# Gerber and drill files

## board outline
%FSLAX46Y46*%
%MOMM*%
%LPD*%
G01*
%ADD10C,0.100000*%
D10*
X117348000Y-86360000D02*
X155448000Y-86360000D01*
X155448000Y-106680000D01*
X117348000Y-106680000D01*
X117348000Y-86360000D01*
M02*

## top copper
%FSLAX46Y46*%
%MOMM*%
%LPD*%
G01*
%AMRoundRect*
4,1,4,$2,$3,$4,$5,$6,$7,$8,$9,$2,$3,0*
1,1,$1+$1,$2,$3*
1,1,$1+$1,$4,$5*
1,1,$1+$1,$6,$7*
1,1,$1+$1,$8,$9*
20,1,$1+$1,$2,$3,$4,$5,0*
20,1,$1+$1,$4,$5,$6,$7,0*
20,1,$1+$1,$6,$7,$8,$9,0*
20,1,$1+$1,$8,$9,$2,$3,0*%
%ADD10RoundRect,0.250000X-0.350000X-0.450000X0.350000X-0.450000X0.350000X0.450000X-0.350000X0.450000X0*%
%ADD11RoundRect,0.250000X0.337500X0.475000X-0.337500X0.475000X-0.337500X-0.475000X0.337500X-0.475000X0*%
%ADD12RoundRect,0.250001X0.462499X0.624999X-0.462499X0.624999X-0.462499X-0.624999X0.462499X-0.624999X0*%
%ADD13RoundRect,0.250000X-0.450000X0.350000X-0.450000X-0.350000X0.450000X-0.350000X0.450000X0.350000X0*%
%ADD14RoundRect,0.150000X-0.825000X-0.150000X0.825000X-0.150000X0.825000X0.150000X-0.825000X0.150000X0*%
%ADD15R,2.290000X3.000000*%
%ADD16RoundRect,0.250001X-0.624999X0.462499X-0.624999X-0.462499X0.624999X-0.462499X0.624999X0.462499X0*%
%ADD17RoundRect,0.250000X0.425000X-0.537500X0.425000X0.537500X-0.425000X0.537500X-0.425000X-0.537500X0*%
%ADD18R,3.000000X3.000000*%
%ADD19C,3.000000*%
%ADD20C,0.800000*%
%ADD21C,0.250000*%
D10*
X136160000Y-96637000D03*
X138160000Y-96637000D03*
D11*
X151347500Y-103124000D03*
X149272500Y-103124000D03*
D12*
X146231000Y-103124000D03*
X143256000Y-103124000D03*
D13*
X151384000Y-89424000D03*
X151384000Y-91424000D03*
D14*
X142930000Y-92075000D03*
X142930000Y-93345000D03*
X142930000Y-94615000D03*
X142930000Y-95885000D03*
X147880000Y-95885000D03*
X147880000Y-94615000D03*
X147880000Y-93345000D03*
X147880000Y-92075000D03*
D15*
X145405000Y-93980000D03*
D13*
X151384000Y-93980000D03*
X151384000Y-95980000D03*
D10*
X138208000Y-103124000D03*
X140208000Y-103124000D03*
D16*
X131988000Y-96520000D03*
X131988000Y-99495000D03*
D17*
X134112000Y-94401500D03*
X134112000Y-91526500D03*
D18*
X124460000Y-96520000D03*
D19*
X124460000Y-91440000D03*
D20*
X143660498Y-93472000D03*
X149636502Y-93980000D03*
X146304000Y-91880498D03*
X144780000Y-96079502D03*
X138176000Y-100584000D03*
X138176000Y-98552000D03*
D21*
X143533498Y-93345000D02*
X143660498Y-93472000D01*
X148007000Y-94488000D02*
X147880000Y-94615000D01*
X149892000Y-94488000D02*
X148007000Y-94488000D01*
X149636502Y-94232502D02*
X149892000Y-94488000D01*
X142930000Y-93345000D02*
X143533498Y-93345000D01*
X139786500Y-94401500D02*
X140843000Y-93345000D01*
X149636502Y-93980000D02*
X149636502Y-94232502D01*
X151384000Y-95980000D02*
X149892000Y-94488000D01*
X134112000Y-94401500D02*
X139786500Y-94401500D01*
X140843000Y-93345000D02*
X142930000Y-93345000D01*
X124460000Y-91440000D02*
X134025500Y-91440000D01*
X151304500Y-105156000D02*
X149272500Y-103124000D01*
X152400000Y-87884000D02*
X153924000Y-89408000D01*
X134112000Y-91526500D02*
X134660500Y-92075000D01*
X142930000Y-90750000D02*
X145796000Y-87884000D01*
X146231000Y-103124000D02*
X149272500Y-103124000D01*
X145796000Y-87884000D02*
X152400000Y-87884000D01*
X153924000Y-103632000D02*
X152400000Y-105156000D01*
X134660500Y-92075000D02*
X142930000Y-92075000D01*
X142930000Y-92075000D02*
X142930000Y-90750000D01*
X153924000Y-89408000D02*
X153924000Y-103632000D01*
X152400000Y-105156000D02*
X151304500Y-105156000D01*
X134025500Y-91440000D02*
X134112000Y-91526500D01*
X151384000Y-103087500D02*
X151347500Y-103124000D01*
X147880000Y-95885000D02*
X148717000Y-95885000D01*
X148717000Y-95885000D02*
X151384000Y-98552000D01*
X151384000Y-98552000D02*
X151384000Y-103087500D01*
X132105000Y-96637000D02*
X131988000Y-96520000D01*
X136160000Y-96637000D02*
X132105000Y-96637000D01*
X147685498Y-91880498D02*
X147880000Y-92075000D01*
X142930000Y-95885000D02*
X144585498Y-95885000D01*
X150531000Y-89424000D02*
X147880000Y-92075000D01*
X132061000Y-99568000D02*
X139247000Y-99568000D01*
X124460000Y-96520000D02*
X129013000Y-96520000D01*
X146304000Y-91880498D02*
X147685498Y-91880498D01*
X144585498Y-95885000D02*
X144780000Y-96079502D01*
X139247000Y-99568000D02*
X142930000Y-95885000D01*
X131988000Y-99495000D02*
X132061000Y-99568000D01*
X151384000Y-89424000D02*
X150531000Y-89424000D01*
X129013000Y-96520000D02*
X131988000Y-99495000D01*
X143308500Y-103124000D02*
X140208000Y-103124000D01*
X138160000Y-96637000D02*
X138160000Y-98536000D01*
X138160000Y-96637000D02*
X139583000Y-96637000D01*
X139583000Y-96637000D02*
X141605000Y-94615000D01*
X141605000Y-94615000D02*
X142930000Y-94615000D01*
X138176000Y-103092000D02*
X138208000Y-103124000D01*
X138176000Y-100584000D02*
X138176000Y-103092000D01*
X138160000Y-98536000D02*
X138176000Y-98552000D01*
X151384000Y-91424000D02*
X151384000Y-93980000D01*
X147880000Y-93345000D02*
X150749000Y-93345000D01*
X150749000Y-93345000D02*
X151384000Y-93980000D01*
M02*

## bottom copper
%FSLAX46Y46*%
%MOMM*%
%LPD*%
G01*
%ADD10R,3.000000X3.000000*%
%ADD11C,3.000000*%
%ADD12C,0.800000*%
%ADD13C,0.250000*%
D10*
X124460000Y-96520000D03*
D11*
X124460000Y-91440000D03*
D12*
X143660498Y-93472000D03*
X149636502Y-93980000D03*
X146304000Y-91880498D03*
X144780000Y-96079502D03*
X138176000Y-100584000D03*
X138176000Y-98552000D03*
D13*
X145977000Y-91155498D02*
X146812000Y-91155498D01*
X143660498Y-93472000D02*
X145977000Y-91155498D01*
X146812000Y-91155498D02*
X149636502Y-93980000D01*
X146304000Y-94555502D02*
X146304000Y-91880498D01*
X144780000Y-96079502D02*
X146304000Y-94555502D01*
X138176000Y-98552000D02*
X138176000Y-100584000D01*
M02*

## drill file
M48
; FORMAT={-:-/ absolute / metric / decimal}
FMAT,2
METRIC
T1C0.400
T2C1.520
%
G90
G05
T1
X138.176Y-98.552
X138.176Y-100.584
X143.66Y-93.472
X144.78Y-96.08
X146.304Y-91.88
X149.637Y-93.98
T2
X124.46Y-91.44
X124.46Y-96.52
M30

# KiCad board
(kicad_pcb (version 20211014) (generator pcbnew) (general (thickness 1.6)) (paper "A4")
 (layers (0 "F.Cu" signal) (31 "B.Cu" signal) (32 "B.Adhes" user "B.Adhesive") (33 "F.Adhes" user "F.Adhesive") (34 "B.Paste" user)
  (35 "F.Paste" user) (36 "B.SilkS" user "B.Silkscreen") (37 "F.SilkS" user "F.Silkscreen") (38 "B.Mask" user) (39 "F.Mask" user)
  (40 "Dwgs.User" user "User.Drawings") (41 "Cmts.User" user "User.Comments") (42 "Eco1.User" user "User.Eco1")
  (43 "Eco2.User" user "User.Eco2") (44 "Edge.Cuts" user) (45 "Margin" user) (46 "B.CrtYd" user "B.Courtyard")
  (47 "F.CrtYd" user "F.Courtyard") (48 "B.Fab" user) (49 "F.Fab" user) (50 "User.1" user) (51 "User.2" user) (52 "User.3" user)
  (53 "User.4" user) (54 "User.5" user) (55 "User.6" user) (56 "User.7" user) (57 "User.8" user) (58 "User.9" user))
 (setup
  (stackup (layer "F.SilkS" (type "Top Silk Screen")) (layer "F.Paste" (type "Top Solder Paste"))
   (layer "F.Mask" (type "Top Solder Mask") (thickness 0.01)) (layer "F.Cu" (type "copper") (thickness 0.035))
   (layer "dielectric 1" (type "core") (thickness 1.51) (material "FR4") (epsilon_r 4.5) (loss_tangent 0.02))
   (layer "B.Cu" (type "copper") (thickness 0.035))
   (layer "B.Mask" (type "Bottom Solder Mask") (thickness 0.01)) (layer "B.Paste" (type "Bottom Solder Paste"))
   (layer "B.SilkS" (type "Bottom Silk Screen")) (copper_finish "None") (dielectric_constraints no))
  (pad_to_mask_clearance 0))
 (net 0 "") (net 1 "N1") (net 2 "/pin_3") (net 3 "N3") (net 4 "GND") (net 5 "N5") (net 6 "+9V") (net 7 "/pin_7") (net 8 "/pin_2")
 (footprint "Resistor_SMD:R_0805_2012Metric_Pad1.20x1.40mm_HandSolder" (layer "F.Cu") (at 137.16 96.637)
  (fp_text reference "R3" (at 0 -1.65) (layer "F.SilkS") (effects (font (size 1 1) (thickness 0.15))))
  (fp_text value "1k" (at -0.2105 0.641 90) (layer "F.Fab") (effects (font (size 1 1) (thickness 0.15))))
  (pad "1" smd roundrect (at -1 0) (size 1.2 1.4) (layers "F.Cu" "F.Paste" "F.Mask") (roundrect_rratio 0.2083333333) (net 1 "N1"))
  (pad "2" smd roundrect (at 1 0) (size 1.2 1.4) (layers "F.Cu" "F.Paste" "F.Mask") (roundrect_rratio 0.2083333333) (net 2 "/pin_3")))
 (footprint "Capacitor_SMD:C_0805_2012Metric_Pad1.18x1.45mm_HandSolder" (layer "F.Cu") (at 150.31 103.124 180)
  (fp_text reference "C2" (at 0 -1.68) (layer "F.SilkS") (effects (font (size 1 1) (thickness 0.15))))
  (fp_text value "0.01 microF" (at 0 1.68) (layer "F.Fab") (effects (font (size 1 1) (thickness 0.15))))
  (pad "1" smd roundrect (at -1.0375 0 180) (size 1.175 1.45) (layers "F.Cu" "F.Paste" "F.Mask") (roundrect_rratio 0.2127659574)
   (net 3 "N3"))
  (pad "2" smd roundrect (at 1.0375 0 180) (size 1.175 1.45) (layers "F.Cu" "F.Paste" "F.Mask") (roundrect_rratio 0.2127659574)
   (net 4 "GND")))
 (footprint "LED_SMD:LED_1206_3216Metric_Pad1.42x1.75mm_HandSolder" (layer "F.Cu") (at 144.7435 103.124 180)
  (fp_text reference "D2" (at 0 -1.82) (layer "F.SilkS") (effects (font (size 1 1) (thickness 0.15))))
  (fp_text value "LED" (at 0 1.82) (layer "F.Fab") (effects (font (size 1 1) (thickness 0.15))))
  (pad "1" smd roundrect (at -1.4875 0 180) (size 1.425 1.75) (layers "F.Cu" "F.Paste" "F.Mask") (roundrect_rratio 0.1754392982)
   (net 4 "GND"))
  (pad "2" smd roundrect (at 1.4875 0 180) (size 1.425 1.75) (layers "F.Cu" "F.Paste" "F.Mask") (roundrect_rratio 0.1754392982) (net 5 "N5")))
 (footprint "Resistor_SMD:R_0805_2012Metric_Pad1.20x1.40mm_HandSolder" (layer "F.Cu") (at 151.384 90.424 -90)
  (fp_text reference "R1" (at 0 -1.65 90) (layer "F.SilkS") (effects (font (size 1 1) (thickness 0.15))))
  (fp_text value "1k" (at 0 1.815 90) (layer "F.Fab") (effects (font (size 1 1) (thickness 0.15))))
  (pad "1" smd roundrect (at -1 0 270) (size 1.2 1.4) (layers "F.Cu" "F.Paste" "F.Mask") (roundrect_rratio 0.2083333333) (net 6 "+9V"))
  (pad "2" smd roundrect (at 1 0 270) (size 1.2 1.4) (layers "F.Cu" "F.Paste" "F.Mask") (roundrect_rratio 0.2083333333) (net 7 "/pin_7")))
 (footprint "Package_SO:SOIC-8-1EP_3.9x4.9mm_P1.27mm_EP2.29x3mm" (layer "F.Cu") (at 145.405 93.98)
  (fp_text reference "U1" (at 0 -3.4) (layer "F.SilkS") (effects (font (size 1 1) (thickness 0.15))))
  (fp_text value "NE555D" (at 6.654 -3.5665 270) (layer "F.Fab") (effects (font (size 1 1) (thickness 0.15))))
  (pad "" smd roundrect (at 0.57 0.75) (size 0.92 1.21) (layers "F.Paste") (roundrect_rratio 0.25))
  (pad "" smd roundrect (at -0.57 0.75) (size 0.92 1.21) (layers "F.Paste") (roundrect_rratio 0.25))
  (pad "" smd roundrect (at -0.57 -0.75) (size 0.92 1.21) (layers "F.Paste") (roundrect_rratio 0.25))
  (pad "" smd roundrect (at 0.57 -0.75) (size 0.92 1.21) (layers "F.Paste") (roundrect_rratio 0.25))
  (pad "1" smd roundrect (at -2.475 -1.905) (size 1.95 0.6) (layers "F.Cu" "F.Paste" "F.Mask") (roundrect_rratio 0.25) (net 4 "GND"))
  (pad "2" smd roundrect (at -2.475 -0.635) (size 1.95 0.6) (layers "F.Cu" "F.Paste" "F.Mask") (roundrect_rratio 0.25) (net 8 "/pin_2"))
  (pad "3" smd roundrect (at -2.475 0.635) (size 1.95 0.6) (layers "F.Cu" "F.Paste" "F.Mask") (roundrect_rratio 0.25) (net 2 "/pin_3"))
  (pad "4" smd roundrect (at -2.475 1.905) (size 1.95 0.6) (layers "F.Cu" "F.Paste" "F.Mask") (roundrect_rratio 0.25) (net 6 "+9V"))
  (pad "5" smd roundrect (at 2.475 1.905) (size 1.95 0.6) (layers "F.Cu" "F.Paste" "F.Mask") (roundrect_rratio 0.25) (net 3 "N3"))
  (pad "6" smd roundrect (at 2.475 0.635) (size 1.95 0.6) (layers "F.Cu" "F.Paste" "F.Mask") (roundrect_rratio 0.25) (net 8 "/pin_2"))
  (pad "7" smd roundrect (at 2.475 -0.635) (size 1.95 0.6) (layers "F.Cu" "F.Paste" "F.Mask") (roundrect_rratio 0.25) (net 7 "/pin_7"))
  (pad "8" smd roundrect (at 2.475 -1.905) (size 1.95 0.6) (layers "F.Cu" "F.Paste" "F.Mask") (roundrect_rratio 0.25) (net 6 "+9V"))
  (pad "9" smd rect (at 0 0) (size 2.29 3) (layers "F.Cu" "F.Mask")))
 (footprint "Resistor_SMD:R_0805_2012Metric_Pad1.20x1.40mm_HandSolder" (layer "F.Cu") (at 151.384 94.98 -90)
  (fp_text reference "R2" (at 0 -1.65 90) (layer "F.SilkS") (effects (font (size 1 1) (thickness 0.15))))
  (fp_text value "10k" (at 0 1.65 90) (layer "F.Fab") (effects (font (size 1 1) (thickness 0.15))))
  (pad "1" smd roundrect (at -1 0 270) (size 1.2 1.4) (layers "F.Cu" "F.Paste" "F.Mask") (roundrect_rratio 0.2083333333) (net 7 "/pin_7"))
  (pad "2" smd roundrect (at 1 0 270) (size 1.2 1.4) (layers "F.Cu" "F.Paste" "F.Mask") (roundrect_rratio 0.2083333333) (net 8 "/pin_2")))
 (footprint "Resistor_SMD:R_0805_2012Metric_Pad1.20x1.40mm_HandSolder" (layer "F.Cu") (at 139.208 103.124)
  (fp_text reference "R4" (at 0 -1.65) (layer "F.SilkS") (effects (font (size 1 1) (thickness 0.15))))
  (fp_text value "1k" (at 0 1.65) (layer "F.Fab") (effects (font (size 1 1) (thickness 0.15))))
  (pad "1" smd roundrect (at -1 0) (size 1.2 1.4) (layers "F.Cu" "F.Paste" "F.Mask") (roundrect_rratio 0.2083333333) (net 2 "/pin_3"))
  (pad "2" smd roundrect (at 1 0) (size 1.2 1.4) (layers "F.Cu" "F.Paste" "F.Mask") (roundrect_rratio 0.2083333333) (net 5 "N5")))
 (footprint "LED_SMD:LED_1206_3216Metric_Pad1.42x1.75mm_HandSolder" (layer "F.Cu") (at 131.988 98.0075 -90)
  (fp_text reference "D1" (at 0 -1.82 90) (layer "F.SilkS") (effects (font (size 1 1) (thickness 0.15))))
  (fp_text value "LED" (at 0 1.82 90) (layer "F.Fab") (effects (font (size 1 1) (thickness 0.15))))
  (pad "1" smd roundrect (at -1.4875 0 270) (size 1.425 1.75) (layers "F.Cu" "F.Paste" "F.Mask") (roundrect_rratio 0.1754392982)
   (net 1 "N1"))
  (pad "2" smd roundrect (at 1.4875 0 270) (size 1.425 1.75) (layers "F.Cu" "F.Paste" "F.Mask") (roundrect_rratio 0.1754392982)
   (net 6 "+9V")))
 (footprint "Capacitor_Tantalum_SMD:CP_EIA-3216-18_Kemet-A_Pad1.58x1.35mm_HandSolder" (layer "F.Cu") (at 134.112 92.964 90)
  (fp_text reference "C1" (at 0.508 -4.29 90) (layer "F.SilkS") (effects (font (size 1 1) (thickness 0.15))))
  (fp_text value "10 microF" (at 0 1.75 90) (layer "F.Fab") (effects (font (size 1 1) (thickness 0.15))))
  (pad "1" smd roundrect (at -1.4375 0 90) (size 1.575 1.35) (layers "F.Cu" "F.Paste" "F.Mask") (roundrect_rratio 0.1851851852)
   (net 8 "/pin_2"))
  (pad "2" smd roundrect (at 1.4375 0 90) (size 1.575 1.35) (layers "F.Cu" "F.Paste" "F.Mask") (roundrect_rratio 0.1851851852) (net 4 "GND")))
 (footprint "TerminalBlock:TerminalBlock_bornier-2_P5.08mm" (layer "F.Cu") (at 124.46 96.52 90)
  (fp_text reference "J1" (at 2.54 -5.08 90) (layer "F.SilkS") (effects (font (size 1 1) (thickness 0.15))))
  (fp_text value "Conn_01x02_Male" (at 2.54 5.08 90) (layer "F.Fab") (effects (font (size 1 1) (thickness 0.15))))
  (pad "1" thru_hole rect (at 0 0 90) (size 3 3) (drill 1.52) (layers *.Cu *.Mask) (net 6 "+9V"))
  (pad "2" thru_hole circle (at 5.08 0 90) (size 3 3) (drill 1.52) (layers *.Cu *.Mask) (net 4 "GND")))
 (gr_rect (start 117.348 86.36) (end 155.448 106.68) (layer "Edge.Cuts") (width 0.1) (fill none))
 (segment (start 143.533498 93.345) (end 143.660498 93.472) (width 0.25) (layer "F.Cu") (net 8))
 (segment (start 148.007 94.488) (end 147.88 94.615) (width 0.25) (layer "F.Cu") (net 8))
 (segment (start 149.892 94.488) (end 148.007 94.488) (width 0.25) (layer "F.Cu") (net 8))
 (segment (start 149.636502 94.232502) (end 149.892 94.488) (width 0.25) (layer "F.Cu") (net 8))
 (segment (start 142.93 93.345) (end 143.533498 93.345) (width 0.25) (layer "F.Cu") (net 8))
 (segment (start 139.7865 94.4015) (end 140.843 93.345) (width 0.25) (layer "F.Cu") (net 8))
 (segment (start 149.636502 93.98) (end 149.636502 94.232502) (width 0.25) (layer "F.Cu") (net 8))
 (segment (start 151.384 95.98) (end 149.892 94.488) (width 0.25) (layer "F.Cu") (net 8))
 (segment (start 134.112 94.4015) (end 139.7865 94.4015) (width 0.25) (layer "F.Cu") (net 8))
 (segment (start 140.843 93.345) (end 142.93 93.345) (width 0.25) (layer "F.Cu") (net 8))
 (via (at 143.660498 93.472) (size 0.8) (drill 0.4) (layers "F.Cu" "B.Cu") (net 8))
 (via (at 149.636502 93.98) (size 0.8) (drill 0.4) (layers "F.Cu" "B.Cu") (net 8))
 (segment (start 145.977 91.155498) (end 146.812 91.155498) (width 0.25) (layer "B.Cu") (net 8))
 (segment (start 143.660498 93.472) (end 145.977 91.155498) (width 0.25) (layer "B.Cu") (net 8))
 (segment (start 146.812 91.155498) (end 149.636502 93.98) (width 0.25) (layer "B.Cu") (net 8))
 (segment (start 124.46 91.44) (end 134.0255 91.44) (width 0.25) (layer "F.Cu") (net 4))
 (segment (start 151.3045 105.156) (end 149.2725 103.124) (width 0.25) (layer "F.Cu") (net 4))
 (segment (start 152.4 87.884) (end 153.924 89.408) (width 0.25) (layer "F.Cu") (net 4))
 (segment (start 134.112 91.5265) (end 134.6605 92.075) (width 0.25) (layer "F.Cu") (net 4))
 (segment (start 142.93 90.75) (end 145.796 87.884) (width 0.25) (layer "F.Cu") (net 4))
 (segment (start 146.231 103.124) (end 149.2725 103.124) (width 0.25) (layer "F.Cu") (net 4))
 (segment (start 145.796 87.884) (end 152.4 87.884) (width 0.25) (layer "F.Cu") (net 4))
 (segment (start 153.924 103.632) (end 152.4 105.156) (width 0.25) (layer "F.Cu") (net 4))
 (segment (start 134.6605 92.075) (end 142.93 92.075) (width 0.25) (layer "F.Cu") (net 4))
 (segment (start 142.93 92.075) (end 142.93 90.75) (width 0.25) (layer "F.Cu") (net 4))
 (segment (start 153.924 89.408) (end 153.924 103.632) (width 0.25) (layer "F.Cu") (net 4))
 (segment (start 152.4 105.156) (end 151.3045 105.156) (width 0.25) (layer "F.Cu") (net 4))
 (segment (start 134.0255 91.44) (end 134.112 91.5265) (width 0.25) (layer "F.Cu") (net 4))
 (segment (start 151.384 103.0875) (end 151.3475 103.124) (width 0.25) (layer "F.Cu") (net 3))
 (segment (start 147.88 95.885) (end 148.717 95.885) (width 0.25) (layer "F.Cu") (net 3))
 (segment (start 148.717 95.885) (end 151.384 98.552) (width 0.25) (layer "F.Cu") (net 3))
 (segment (start 151.384 98.552) (end 151.384 103.0875) (width 0.25) (layer "F.Cu") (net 3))
 (segment (start 132.105 96.637) (end 131.988 96.52) (width 0.25) (layer "F.Cu") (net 1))
 (segment (start 136.16 96.637) (end 132.105 96.637) (width 0.25) (layer "F.Cu") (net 1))
 (segment (start 147.685498 91.880498) (end 147.88 92.075) (width 0.25) (layer "F.Cu") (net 6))
 (segment (start 142.93 95.885) (end 144.585498 95.885) (width 0.25) (layer "F.Cu") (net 6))
 (segment (start 150.531 89.424) (end 147.88 92.075) (width 0.25) (layer "F.Cu") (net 6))
 (segment (start 132.061 99.568) (end 139.247 99.568) (width 0.25) (layer "F.Cu") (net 6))
 (segment (start 124.46 96.52) (end 129.013 96.52) (width 0.25) (layer "F.Cu") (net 6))
 (segment (start 146.304 91.880498) (end 147.685498 91.880498) (width 0.25) (layer "F.Cu") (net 6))
 (segment (start 144.585498 95.885) (end 144.78 96.079502) (width 0.25) (layer "F.Cu") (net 6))
 (segment (start 139.247 99.568) (end 142.93 95.885) (width 0.25) (layer "F.Cu") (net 6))
 (segment (start 131.988 99.495) (end 132.061 99.568) (width 0.25) (layer "F.Cu") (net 6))
 (segment (start 151.384 89.424) (end 150.531 89.424) (width 0.25) (layer "F.Cu") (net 6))
 (segment (start 129.013 96.52) (end 131.988 99.495) (width 0.25) (layer "F.Cu") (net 6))
 (via (at 146.304 91.880498) (size 0.8) (drill 0.4) (layers "F.Cu" "B.Cu") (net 6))
 (via (at 144.78 96.079502) (size 0.8) (drill 0.4) (layers "F.Cu" "B.Cu") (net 6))
 (segment (start 146.304 94.555502) (end 146.304 91.880498) (width 0.25) (layer "B.Cu") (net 6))
 (segment (start 144.78 96.079502) (end 146.304 94.555502) (width 0.25) (layer "B.Cu") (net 6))
 (segment (start 143.3085 103.124) (end 140.208 103.124) (width 0.25) (layer "F.Cu") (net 5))
 (segment (start 138.16 96.637) (end 138.16 98.536) (width 0.25) (layer "F.Cu") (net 2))
 (segment (start 138.16 96.637) (end 139.583 96.637) (width 0.25) (layer "F.Cu") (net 2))
 (segment (start 139.583 96.637) (end 141.605 94.615) (width 0.25) (layer "F.Cu") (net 2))
 (segment (start 141.605 94.615) (end 142.93 94.615) (width 0.25) (layer "F.Cu") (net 2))
 (segment (start 138.176 103.092) (end 138.208 103.124) (width 0.25) (layer "F.Cu") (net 2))
 (segment (start 138.176 100.584) (end 138.176 103.092) (width 0.25) (layer "F.Cu") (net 2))
 (segment (start 138.16 98.536) (end 138.176 98.552) (width 0.25) (layer "F.Cu") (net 2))
 (via (at 138.176 100.584) (size 0.8) (drill 0.4) (layers "F.Cu" "B.Cu") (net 2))
 (via (at 138.176 98.552) (size 0.8) (drill 0.4) (layers "F.Cu" "B.Cu") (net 2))
 (segment (start 138.176 98.552) (end 138.176 100.584) (width 0.25) (layer "B.Cu") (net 2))
 (segment (start 151.384 91.424) (end 151.384 93.98) (width 0.25) (layer "F.Cu") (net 7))
 (segment (start 147.88 93.345) (end 150.749 93.345) (width 0.25) (layer "F.Cu") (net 7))
 (segment (start 150.749 93.345) (end 151.384 93.98) (width 0.25) (layer "F.Cu") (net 7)))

